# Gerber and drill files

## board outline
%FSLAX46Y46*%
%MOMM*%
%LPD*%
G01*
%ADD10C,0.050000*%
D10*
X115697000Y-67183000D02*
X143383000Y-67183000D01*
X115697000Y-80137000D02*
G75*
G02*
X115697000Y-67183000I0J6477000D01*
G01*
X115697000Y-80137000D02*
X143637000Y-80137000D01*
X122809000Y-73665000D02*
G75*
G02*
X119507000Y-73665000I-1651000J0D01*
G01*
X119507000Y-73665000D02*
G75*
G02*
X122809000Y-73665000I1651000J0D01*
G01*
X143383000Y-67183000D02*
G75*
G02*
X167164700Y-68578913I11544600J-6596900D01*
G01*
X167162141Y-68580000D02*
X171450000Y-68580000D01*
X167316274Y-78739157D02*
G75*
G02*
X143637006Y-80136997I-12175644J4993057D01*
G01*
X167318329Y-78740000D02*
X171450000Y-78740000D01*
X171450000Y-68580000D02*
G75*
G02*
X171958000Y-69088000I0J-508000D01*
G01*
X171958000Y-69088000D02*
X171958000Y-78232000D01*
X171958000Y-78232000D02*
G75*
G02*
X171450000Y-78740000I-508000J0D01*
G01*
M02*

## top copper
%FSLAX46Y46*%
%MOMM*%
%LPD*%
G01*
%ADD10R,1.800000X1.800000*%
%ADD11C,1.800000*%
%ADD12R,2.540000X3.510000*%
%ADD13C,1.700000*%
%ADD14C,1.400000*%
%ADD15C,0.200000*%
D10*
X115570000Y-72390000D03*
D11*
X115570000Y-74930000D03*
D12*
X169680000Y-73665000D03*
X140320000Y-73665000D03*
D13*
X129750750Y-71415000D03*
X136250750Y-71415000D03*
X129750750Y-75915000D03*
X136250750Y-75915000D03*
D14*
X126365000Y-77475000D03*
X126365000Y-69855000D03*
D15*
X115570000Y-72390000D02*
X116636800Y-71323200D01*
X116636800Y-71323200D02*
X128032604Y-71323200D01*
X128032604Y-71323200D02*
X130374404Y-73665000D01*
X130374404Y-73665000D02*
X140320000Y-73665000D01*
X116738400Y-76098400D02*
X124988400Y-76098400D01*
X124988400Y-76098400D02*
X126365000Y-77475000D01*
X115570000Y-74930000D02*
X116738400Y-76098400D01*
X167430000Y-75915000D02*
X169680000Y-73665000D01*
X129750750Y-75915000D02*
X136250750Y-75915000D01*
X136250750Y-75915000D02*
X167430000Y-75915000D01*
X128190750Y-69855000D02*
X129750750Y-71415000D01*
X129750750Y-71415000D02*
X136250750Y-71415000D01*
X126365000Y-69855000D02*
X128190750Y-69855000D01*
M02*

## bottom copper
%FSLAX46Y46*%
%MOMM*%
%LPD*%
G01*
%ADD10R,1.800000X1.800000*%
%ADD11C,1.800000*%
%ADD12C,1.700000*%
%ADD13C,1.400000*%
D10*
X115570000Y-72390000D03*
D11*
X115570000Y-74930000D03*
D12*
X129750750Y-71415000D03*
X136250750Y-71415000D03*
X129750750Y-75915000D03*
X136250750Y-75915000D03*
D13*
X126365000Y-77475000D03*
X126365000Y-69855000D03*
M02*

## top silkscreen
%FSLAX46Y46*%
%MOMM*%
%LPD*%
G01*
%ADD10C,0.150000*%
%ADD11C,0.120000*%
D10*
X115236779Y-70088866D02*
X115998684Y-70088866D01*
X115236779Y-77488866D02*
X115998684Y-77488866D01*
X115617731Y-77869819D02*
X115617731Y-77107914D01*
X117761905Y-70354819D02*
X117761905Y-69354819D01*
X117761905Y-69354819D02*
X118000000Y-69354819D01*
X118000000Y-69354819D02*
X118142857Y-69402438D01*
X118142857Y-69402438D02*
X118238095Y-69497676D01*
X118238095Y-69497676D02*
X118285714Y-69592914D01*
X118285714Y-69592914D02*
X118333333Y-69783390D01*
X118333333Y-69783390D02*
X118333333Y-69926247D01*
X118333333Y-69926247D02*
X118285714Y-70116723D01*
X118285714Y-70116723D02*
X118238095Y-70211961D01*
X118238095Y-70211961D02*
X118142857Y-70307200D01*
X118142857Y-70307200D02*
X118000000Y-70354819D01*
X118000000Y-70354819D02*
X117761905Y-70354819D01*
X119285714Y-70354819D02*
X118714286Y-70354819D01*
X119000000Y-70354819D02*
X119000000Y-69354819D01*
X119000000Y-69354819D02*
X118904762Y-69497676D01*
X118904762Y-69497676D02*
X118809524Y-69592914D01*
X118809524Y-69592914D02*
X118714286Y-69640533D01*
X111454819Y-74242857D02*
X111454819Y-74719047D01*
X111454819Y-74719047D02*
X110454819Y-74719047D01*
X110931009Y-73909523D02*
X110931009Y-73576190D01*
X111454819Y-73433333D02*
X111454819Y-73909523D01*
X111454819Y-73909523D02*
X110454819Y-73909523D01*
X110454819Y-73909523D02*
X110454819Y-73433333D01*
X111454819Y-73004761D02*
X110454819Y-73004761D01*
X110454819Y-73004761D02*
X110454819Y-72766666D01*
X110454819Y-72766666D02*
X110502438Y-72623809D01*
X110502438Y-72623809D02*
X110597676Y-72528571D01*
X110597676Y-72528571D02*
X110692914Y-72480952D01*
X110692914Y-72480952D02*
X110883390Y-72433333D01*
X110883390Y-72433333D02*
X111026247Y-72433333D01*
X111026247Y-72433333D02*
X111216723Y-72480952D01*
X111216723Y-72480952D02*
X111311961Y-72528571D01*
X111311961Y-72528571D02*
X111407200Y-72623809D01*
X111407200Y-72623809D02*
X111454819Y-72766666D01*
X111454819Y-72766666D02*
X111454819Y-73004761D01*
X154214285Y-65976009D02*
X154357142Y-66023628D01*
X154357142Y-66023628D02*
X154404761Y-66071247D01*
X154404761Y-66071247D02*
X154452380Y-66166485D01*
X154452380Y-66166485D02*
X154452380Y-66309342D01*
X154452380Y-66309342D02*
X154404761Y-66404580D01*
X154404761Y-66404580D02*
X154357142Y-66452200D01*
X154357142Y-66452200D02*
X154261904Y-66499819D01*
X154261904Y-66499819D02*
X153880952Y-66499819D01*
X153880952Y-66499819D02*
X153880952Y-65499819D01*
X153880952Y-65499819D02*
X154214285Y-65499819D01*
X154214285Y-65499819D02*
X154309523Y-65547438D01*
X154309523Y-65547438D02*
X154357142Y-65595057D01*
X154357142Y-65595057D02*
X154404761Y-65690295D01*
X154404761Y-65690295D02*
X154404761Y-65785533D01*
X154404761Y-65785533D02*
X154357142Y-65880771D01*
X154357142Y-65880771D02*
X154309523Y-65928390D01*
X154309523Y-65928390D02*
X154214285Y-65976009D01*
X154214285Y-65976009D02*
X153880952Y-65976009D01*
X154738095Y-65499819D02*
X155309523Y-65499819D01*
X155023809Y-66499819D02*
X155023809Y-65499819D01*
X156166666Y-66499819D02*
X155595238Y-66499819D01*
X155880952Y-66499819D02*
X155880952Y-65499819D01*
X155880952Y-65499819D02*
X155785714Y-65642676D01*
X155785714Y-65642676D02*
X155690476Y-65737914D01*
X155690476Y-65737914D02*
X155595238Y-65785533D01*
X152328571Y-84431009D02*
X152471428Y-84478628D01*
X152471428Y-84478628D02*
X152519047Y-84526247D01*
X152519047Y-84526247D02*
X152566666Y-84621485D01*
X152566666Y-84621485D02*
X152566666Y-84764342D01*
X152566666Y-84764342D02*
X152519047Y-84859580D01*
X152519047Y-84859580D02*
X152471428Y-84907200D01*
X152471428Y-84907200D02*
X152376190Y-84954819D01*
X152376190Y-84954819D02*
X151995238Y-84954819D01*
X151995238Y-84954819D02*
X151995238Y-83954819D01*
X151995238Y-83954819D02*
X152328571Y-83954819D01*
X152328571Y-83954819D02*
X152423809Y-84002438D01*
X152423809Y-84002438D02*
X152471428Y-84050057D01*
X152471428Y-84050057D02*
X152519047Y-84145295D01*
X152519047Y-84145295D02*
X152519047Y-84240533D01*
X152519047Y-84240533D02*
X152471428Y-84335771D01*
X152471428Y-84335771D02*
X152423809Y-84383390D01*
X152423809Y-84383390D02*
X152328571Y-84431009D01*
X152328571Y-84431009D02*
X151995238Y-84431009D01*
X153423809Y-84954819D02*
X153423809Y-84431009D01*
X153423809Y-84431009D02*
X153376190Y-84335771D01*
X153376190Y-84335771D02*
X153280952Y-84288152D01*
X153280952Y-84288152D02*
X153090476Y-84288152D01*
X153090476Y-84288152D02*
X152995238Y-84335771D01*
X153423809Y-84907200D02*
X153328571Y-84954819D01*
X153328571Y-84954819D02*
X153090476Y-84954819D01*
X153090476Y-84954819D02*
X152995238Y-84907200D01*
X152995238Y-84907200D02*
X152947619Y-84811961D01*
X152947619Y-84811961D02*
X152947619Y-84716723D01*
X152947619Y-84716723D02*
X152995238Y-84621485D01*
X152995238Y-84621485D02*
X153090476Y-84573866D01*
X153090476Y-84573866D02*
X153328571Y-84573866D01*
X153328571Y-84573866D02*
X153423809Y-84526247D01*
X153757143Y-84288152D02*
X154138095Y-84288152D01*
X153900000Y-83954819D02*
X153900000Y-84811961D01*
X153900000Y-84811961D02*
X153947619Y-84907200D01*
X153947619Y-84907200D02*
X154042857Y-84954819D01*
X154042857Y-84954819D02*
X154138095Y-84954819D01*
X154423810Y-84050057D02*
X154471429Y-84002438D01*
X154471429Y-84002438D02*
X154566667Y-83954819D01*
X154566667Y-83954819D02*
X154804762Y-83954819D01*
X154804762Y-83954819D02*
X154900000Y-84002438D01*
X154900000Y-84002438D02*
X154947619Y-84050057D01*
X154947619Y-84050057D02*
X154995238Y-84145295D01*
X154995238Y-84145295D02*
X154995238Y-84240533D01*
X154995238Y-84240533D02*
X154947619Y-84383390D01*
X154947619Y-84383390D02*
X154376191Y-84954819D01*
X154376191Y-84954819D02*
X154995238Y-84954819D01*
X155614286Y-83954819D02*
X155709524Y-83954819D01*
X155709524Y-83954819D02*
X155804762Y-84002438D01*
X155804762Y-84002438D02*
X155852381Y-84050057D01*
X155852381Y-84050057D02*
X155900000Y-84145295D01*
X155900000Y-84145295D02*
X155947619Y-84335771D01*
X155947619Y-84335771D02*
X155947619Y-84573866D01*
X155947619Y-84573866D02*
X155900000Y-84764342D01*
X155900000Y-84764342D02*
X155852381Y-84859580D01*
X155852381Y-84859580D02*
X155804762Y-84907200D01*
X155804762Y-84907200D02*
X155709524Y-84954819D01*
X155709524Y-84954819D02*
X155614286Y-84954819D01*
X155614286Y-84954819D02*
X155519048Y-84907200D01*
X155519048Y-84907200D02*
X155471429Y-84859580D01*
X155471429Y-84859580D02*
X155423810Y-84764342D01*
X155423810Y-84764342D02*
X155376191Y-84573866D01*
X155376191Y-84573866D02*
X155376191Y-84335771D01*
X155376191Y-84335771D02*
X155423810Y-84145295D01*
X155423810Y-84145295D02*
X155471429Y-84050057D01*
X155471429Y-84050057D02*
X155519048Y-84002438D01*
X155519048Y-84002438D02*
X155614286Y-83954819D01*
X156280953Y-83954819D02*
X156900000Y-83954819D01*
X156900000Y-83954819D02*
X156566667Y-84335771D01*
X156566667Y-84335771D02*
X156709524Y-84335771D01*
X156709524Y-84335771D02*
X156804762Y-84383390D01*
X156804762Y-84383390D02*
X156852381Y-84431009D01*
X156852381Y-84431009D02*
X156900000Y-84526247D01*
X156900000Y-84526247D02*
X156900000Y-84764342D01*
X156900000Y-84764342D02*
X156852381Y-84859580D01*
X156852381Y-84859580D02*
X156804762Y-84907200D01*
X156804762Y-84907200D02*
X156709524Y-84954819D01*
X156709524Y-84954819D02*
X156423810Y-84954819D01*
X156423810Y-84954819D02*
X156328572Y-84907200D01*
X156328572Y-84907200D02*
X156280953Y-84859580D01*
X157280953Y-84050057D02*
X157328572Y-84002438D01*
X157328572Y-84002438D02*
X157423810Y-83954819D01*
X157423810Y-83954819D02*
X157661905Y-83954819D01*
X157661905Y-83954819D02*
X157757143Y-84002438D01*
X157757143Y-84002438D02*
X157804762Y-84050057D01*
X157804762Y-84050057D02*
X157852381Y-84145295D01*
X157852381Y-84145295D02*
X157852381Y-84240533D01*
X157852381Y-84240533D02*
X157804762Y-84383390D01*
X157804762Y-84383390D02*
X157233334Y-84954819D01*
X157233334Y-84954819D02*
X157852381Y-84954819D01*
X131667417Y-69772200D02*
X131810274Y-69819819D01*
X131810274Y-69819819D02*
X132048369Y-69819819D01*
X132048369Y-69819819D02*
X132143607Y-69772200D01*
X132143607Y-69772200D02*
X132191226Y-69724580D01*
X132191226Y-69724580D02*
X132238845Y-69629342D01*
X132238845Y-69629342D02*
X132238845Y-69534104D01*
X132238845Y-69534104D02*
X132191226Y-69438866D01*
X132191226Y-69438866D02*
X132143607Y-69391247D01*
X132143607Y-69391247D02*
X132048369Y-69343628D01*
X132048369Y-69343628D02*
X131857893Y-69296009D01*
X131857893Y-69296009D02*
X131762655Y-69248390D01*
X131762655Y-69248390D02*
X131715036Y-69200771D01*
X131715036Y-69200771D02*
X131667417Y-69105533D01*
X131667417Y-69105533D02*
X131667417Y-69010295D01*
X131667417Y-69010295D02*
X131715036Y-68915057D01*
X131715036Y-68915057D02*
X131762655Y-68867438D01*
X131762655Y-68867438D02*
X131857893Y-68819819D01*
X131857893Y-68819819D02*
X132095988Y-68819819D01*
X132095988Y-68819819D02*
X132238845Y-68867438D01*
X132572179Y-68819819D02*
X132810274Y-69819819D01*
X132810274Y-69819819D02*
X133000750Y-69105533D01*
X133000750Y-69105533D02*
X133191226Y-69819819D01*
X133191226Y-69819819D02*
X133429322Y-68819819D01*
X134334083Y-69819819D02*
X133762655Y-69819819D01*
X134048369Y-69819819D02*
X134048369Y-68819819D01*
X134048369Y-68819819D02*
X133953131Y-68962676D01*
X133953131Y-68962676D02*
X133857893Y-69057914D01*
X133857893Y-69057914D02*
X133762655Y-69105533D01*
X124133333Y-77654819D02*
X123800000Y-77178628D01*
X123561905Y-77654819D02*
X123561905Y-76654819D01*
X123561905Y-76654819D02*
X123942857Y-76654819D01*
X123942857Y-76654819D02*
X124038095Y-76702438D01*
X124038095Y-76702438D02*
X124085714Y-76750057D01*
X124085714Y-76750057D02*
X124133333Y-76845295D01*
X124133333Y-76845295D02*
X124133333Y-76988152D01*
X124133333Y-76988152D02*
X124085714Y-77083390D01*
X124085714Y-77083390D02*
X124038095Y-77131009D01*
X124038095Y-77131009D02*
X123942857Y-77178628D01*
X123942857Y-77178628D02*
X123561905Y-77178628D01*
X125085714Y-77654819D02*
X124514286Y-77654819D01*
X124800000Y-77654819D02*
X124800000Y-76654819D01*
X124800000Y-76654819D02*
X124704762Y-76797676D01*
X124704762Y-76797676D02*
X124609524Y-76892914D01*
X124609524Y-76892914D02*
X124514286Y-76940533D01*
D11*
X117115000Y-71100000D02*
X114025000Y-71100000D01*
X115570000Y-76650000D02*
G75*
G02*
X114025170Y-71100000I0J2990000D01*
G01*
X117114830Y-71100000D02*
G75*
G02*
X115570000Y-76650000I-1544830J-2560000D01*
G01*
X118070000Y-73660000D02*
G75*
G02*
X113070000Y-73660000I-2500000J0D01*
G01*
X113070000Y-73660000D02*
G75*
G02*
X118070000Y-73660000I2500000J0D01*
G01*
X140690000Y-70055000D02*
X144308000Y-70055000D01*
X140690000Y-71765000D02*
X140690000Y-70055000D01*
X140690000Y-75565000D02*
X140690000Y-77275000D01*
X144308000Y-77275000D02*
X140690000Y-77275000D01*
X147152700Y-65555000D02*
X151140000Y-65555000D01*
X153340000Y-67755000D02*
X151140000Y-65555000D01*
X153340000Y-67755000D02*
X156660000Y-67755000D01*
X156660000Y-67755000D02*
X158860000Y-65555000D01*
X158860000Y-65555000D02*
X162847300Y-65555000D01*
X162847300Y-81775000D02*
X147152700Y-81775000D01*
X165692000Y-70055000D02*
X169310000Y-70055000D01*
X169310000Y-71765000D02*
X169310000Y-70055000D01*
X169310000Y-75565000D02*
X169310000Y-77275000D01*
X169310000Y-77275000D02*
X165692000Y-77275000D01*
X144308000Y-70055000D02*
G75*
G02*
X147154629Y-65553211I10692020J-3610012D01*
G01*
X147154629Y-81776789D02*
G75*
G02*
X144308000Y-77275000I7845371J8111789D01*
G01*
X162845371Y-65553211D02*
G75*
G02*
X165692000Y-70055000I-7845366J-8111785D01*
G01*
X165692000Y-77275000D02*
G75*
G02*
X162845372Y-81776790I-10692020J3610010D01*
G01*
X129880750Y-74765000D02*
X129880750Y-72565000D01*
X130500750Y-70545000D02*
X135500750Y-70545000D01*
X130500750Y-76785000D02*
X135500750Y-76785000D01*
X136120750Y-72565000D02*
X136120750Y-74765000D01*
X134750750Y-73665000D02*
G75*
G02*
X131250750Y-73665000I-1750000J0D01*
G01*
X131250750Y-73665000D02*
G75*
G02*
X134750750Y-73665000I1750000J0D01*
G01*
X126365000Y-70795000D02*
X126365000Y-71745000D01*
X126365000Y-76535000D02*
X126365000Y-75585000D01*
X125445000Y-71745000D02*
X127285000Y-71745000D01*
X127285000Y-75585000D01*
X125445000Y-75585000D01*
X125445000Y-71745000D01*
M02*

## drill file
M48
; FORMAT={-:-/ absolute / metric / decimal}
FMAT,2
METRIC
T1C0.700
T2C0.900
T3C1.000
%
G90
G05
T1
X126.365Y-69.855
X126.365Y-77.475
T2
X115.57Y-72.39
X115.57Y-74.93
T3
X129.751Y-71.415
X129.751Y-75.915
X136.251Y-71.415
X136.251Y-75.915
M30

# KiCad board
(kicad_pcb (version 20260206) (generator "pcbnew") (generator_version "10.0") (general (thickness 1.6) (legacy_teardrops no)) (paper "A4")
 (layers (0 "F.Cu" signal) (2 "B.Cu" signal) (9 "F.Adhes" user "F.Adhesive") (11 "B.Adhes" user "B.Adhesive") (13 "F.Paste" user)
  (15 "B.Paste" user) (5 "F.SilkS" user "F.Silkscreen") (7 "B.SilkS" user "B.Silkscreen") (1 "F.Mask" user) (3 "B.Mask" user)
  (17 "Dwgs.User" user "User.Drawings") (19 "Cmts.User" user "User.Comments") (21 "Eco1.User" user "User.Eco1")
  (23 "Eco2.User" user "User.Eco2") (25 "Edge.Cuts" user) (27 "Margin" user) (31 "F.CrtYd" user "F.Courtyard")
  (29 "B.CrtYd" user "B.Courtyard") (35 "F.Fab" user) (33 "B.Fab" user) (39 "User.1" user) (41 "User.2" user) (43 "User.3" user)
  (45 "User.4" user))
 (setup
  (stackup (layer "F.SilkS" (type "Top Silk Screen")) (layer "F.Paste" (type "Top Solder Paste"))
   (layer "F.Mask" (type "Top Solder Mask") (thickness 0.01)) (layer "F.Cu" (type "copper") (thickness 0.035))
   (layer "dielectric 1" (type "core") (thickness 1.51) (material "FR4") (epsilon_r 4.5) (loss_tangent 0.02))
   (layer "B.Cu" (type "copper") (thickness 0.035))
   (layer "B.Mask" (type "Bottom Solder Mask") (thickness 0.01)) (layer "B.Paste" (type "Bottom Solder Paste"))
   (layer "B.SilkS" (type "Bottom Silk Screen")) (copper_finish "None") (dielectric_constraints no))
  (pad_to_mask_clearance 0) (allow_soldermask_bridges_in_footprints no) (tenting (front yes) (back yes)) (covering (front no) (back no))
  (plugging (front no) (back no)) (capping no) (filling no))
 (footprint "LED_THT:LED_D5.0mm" (layer "F.Cu") (at 115.57 72.39 -90)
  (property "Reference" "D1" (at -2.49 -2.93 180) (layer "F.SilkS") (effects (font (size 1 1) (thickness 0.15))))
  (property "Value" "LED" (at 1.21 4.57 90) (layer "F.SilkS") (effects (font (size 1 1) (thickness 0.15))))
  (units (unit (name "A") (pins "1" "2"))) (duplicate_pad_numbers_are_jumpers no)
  (fp_line (start -1.29 -1.545) (end -1.29 1.545) (stroke (width 0.12) (type solid)) (layer "F.SilkS"))
  (fp_arc (start 4.26 0) (mid 2.071779 2.880495) (end -1.29 1.54483) (stroke (width 0.12) (type solid)) (layer "F.SilkS"))
  (fp_arc (start -1.29 -1.54483) (mid 2.071779 -2.880495) (end 4.26 0) (stroke (width 0.12) (type solid)) (layer "F.SilkS"))
  (fp_circle (center 1.27 0) (end 3.77 0) (stroke (width 0.12) (type solid)) (fill no) (layer "F.SilkS"))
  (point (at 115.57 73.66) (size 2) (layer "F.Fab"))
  (pad "1" thru_hole rect (at 0 0 270) (size 1.8 1.8) (drill 0.9) (layers "*.Cu" "*.Mask") (remove_unused_layers no) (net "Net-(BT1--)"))
  (pad "2" thru_hole circle (at 2.54 0 270) (size 1.8 1.8) (drill 0.9) (layers "*.Cu" "*.Mask") (remove_unused_layers no) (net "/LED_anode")))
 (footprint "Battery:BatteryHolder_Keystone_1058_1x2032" (layer "F.Cu") (at 155 73.665 180)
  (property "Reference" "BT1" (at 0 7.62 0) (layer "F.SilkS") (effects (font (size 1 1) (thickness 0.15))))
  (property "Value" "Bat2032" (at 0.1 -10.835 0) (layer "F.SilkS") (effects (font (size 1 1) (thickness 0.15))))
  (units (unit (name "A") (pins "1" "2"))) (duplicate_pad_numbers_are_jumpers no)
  (fp_line (start 14.31 3.61) (end 10.692 3.61) (stroke (width 0.12) (type solid)) (layer "F.SilkS"))
  (fp_line (start 14.31 1.9) (end 14.31 3.61) (stroke (width 0.12) (type solid)) (layer "F.SilkS"))
  (fp_line (start 14.31 -1.9) (end 14.31 -3.61) (stroke (width 0.12) (type solid)) (layer "F.SilkS"))
  (fp_line (start 10.692 -3.61) (end 14.31 -3.61) (stroke (width 0.12) (type solid)) (layer "F.SilkS"))
  (fp_line (start 7.8473 8.11) (end 3.86 8.11) (stroke (width 0.12) (type solid)) (layer "F.SilkS"))
  (fp_line (start 1.66 5.91) (end 3.86 8.11) (stroke (width 0.12) (type solid)) (layer "F.SilkS"))
  (fp_line (start 1.66 5.91) (end -1.66 5.91) (stroke (width 0.12) (type solid)) (layer "F.SilkS"))
  (fp_line (start -1.66 5.91) (end -3.86 8.11) (stroke (width 0.12) (type solid)) (layer "F.SilkS"))
  (fp_line (start -3.86 8.11) (end -7.8473 8.11) (stroke (width 0.12) (type solid)) (layer "F.SilkS"))
  (fp_line (start -7.8473 -8.11) (end 7.8473 -8.11) (stroke (width 0.12) (type solid)) (layer "F.SilkS"))
  (fp_line (start -10.692 3.61) (end -14.31 3.61) (stroke (width 0.12) (type solid)) (layer "F.SilkS"))
  (fp_line (start -14.31 1.9) (end -14.31 3.61) (stroke (width 0.12) (type solid)) (layer "F.SilkS"))
  (fp_line (start -14.31 -1.9) (end -14.31 -3.61) (stroke (width 0.12) (type solid)) (layer "F.SilkS"))
  (fp_line (start -14.31 -3.61) (end -10.692 -3.61) (stroke (width 0.12) (type solid)) (layer "F.SilkS"))
  (fp_arc (start 10.692 3.61) (mid 9.538084 6.031244) (end 7.845371 8.111789) (stroke (width 0.12) (type solid)) (layer "F.SilkS"))
  (fp_arc (start 7.845371 -8.111789) (mid 9.538085 -6.031244) (end 10.692 -3.61) (stroke (width 0.12) (type solid)) (layer "F.SilkS"))
  (fp_arc (start -7.845371 8.111789) (mid -9.538085 6.031244) (end -10.692 3.61) (stroke (width 0.12) (type solid)) (layer "F.SilkS"))
  (fp_arc (start -10.692 -3.61) (mid -9.538084 -6.031244) (end -7.845371 -8.111789) (stroke (width 0.12) (type solid)) (layer "F.SilkS"))
  (pad "1" smd rect (at -14.68 0 180) (size 2.54 3.51) (layers "F.Cu" "F.Mask" "F.Paste") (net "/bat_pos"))
  (pad "2" smd rect (at 14.68 0 180) (size 2.54 3.51) (layers "F.Cu" "F.Mask" "F.Paste") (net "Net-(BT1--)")))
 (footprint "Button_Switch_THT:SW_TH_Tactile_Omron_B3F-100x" (layer "F.Cu") (at 129.75075 71.415)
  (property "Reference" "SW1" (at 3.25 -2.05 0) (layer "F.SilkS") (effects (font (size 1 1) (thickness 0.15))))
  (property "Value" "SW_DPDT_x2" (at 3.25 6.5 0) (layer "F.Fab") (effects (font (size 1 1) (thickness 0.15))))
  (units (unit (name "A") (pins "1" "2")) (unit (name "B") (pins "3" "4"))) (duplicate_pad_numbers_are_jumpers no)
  (fp_line (start 0.13 3.35) (end 0.13 1.15) (stroke (width 0.12) (type solid)) (layer "F.SilkS"))
  (fp_line (start 0.75 -0.87) (end 5.75 -0.87) (stroke (width 0.12) (type solid)) (layer "F.SilkS"))
  (fp_line (start 0.75 5.37) (end 5.75 5.37) (stroke (width 0.12) (type solid)) (layer "F.SilkS"))
  (fp_line (start 6.37 1.15) (end 6.37 3.35) (stroke (width 0.12) (type solid)) (layer "F.SilkS"))
  (fp_circle (center 3.25 2.25) (end 5 2.25) (stroke (width 0.12) (type solid)) (fill no) (layer "F.SilkS"))
  (pad "1" thru_hole circle (at 0 0) (size 1.7 1.7) (drill 1) (layers "*.Cu" "*.Mask") (remove_unused_layers no) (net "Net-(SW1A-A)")
   (thermal_bridge_angle 90))
  (pad "1" thru_hole circle (at 6.5 0) (size 1.7 1.7) (drill 1) (layers "*.Cu" "*.Mask") (remove_unused_layers no) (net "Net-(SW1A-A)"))
  (pad "2" thru_hole circle (at 0 4.5) (size 1.7 1.7) (drill 1) (layers "*.Cu" "*.Mask") (remove_unused_layers no) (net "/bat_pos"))
  (pad "2" thru_hole circle (at 6.5 4.5) (size 1.7 1.7) (drill 1) (layers "*.Cu" "*.Mask") (remove_unused_layers no) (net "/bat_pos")))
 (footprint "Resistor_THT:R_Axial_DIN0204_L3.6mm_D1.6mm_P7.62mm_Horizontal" (layer "F.Cu") (at 126.365 77.475 90)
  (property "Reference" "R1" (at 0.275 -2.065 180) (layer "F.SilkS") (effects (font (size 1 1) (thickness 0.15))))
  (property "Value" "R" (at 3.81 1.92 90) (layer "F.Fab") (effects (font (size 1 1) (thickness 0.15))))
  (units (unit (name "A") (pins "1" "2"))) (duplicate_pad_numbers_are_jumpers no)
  (fp_line (start 6.68 0) (end 5.73 0) (stroke (width 0.12) (type solid)) (layer "F.SilkS"))
  (fp_line (start 0.94 0) (end 1.89 0) (stroke (width 0.12) (type solid)) (layer "F.SilkS"))
  (fp_rect (start 1.89 -0.92) (end 5.73 0.92) (stroke (width 0.12) (type solid)) (fill no) (layer "F.SilkS"))
  (pad "1" thru_hole circle (at 0 0 90) (size 1.4 1.4) (drill 0.7) (layers "*.Cu" "*.Mask") (remove_unused_layers no) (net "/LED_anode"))
  (pad "2" thru_hole circle (at 7.62 0 90) (size 1.4 1.4) (drill 0.7) (layers "*.Cu" "*.Mask") (remove_unused_layers no)
   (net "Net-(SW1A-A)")))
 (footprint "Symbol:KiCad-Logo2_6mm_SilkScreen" (layer "B.Cu") (at 154.94 70.612 180)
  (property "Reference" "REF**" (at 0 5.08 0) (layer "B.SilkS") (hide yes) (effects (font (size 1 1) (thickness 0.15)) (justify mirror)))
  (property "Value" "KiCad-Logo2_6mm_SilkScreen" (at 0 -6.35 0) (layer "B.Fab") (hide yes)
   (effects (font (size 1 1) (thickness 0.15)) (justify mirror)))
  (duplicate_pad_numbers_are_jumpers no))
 (gr_line (start 115.697 67.183) (end 143.383 67.183) (stroke (width 0.05) (type default)) (layer "Edge.Cuts"))
 (gr_arc (start 115.697 80.137) (mid 109.22 73.66) (end 115.697 67.183) (stroke (width 0.05) (type default)) (layer "Edge.Cuts"))
 (gr_line (start 115.697 80.137) (end 143.637 80.137) (stroke (width 0.05) (type default)) (layer "Edge.Cuts"))
 (gr_circle (center 121.158 73.665) (end 122.809 73.665) (stroke (width 0.05) (type default)) (fill no) (layer "Edge.Cuts"))
 (gr_arc (start 143.383 67.183) (mid 155.70672 60.506257) (end 167.164694 68.578915) (stroke (width 0.05) (type default))
  (layer "Edge.Cuts"))
 (gr_line (start 167.162141 68.58) (end 171.45 68.58) (stroke (width 0.05) (type default)) (layer "Edge.Cuts"))
 (gr_arc (start 167.316274 78.739157) (mid 155.916122 86.882902) (end 143.637 80.137) (stroke (width 0.05) (type default))
  (layer "Edge.Cuts"))
 (gr_line (start 167.318329 78.74) (end 171.45 78.74) (stroke (width 0.05) (type default)) (layer "Edge.Cuts"))
 (gr_arc (start 171.45 68.58) (mid 171.80921 68.72879) (end 171.958 69.088) (stroke (width 0.05) (type default)) (layer "Edge.Cuts"))
 (gr_line (start 171.958 69.088) (end 171.958 78.232) (stroke (width 0.05) (type default)) (layer "Edge.Cuts"))
 (gr_arc (start 171.958 78.232) (mid 171.80921 78.59121) (end 171.45 78.74) (stroke (width 0.05) (type default)) (layer "Edge.Cuts"))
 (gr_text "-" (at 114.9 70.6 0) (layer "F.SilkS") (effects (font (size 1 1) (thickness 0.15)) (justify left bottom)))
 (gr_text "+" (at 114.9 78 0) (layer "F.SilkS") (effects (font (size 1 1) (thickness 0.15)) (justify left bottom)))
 (segment (start 115.57 72.39) (end 116.6368 71.3232) (width 0.2) (layer "F.Cu") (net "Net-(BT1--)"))
 (segment (start 116.6368 71.3232) (end 128.032604 71.3232) (width 0.2) (layer "F.Cu") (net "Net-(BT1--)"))
 (segment (start 128.032604 71.3232) (end 130.374404 73.665) (width 0.2) (layer "F.Cu") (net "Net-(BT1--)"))
 (segment (start 130.374404 73.665) (end 140.32 73.665) (width 0.2) (layer "F.Cu") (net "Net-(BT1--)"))
 (segment (start 116.7384 76.0984) (end 124.9884 76.0984) (width 0.2) (layer "F.Cu") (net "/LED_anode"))
 (segment (start 124.9884 76.0984) (end 126.365 77.475) (width 0.2) (layer "F.Cu") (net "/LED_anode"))
 (segment (start 115.57 74.93) (end 116.7384 76.0984) (width 0.2) (layer "F.Cu") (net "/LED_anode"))
 (segment (start 167.43 75.915) (end 169.68 73.665) (width 0.2) (layer "F.Cu") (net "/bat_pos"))
 (segment (start 129.75075 75.915) (end 136.25075 75.915) (width 0.2) (layer "F.Cu") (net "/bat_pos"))
 (segment (start 136.25075 75.915) (end 167.43 75.915) (width 0.2) (layer "F.Cu") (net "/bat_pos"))
 (segment (start 128.19075 69.855) (end 129.75075 71.415) (width 0.2) (layer "F.Cu") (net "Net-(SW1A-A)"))
 (segment (start 129.75075 71.415) (end 136.25075 71.415) (width 0.2) (layer "F.Cu") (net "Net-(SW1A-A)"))
 (segment (start 126.365 69.855) (end 128.19075 69.855) (width 0.2) (layer "F.Cu") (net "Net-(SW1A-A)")))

